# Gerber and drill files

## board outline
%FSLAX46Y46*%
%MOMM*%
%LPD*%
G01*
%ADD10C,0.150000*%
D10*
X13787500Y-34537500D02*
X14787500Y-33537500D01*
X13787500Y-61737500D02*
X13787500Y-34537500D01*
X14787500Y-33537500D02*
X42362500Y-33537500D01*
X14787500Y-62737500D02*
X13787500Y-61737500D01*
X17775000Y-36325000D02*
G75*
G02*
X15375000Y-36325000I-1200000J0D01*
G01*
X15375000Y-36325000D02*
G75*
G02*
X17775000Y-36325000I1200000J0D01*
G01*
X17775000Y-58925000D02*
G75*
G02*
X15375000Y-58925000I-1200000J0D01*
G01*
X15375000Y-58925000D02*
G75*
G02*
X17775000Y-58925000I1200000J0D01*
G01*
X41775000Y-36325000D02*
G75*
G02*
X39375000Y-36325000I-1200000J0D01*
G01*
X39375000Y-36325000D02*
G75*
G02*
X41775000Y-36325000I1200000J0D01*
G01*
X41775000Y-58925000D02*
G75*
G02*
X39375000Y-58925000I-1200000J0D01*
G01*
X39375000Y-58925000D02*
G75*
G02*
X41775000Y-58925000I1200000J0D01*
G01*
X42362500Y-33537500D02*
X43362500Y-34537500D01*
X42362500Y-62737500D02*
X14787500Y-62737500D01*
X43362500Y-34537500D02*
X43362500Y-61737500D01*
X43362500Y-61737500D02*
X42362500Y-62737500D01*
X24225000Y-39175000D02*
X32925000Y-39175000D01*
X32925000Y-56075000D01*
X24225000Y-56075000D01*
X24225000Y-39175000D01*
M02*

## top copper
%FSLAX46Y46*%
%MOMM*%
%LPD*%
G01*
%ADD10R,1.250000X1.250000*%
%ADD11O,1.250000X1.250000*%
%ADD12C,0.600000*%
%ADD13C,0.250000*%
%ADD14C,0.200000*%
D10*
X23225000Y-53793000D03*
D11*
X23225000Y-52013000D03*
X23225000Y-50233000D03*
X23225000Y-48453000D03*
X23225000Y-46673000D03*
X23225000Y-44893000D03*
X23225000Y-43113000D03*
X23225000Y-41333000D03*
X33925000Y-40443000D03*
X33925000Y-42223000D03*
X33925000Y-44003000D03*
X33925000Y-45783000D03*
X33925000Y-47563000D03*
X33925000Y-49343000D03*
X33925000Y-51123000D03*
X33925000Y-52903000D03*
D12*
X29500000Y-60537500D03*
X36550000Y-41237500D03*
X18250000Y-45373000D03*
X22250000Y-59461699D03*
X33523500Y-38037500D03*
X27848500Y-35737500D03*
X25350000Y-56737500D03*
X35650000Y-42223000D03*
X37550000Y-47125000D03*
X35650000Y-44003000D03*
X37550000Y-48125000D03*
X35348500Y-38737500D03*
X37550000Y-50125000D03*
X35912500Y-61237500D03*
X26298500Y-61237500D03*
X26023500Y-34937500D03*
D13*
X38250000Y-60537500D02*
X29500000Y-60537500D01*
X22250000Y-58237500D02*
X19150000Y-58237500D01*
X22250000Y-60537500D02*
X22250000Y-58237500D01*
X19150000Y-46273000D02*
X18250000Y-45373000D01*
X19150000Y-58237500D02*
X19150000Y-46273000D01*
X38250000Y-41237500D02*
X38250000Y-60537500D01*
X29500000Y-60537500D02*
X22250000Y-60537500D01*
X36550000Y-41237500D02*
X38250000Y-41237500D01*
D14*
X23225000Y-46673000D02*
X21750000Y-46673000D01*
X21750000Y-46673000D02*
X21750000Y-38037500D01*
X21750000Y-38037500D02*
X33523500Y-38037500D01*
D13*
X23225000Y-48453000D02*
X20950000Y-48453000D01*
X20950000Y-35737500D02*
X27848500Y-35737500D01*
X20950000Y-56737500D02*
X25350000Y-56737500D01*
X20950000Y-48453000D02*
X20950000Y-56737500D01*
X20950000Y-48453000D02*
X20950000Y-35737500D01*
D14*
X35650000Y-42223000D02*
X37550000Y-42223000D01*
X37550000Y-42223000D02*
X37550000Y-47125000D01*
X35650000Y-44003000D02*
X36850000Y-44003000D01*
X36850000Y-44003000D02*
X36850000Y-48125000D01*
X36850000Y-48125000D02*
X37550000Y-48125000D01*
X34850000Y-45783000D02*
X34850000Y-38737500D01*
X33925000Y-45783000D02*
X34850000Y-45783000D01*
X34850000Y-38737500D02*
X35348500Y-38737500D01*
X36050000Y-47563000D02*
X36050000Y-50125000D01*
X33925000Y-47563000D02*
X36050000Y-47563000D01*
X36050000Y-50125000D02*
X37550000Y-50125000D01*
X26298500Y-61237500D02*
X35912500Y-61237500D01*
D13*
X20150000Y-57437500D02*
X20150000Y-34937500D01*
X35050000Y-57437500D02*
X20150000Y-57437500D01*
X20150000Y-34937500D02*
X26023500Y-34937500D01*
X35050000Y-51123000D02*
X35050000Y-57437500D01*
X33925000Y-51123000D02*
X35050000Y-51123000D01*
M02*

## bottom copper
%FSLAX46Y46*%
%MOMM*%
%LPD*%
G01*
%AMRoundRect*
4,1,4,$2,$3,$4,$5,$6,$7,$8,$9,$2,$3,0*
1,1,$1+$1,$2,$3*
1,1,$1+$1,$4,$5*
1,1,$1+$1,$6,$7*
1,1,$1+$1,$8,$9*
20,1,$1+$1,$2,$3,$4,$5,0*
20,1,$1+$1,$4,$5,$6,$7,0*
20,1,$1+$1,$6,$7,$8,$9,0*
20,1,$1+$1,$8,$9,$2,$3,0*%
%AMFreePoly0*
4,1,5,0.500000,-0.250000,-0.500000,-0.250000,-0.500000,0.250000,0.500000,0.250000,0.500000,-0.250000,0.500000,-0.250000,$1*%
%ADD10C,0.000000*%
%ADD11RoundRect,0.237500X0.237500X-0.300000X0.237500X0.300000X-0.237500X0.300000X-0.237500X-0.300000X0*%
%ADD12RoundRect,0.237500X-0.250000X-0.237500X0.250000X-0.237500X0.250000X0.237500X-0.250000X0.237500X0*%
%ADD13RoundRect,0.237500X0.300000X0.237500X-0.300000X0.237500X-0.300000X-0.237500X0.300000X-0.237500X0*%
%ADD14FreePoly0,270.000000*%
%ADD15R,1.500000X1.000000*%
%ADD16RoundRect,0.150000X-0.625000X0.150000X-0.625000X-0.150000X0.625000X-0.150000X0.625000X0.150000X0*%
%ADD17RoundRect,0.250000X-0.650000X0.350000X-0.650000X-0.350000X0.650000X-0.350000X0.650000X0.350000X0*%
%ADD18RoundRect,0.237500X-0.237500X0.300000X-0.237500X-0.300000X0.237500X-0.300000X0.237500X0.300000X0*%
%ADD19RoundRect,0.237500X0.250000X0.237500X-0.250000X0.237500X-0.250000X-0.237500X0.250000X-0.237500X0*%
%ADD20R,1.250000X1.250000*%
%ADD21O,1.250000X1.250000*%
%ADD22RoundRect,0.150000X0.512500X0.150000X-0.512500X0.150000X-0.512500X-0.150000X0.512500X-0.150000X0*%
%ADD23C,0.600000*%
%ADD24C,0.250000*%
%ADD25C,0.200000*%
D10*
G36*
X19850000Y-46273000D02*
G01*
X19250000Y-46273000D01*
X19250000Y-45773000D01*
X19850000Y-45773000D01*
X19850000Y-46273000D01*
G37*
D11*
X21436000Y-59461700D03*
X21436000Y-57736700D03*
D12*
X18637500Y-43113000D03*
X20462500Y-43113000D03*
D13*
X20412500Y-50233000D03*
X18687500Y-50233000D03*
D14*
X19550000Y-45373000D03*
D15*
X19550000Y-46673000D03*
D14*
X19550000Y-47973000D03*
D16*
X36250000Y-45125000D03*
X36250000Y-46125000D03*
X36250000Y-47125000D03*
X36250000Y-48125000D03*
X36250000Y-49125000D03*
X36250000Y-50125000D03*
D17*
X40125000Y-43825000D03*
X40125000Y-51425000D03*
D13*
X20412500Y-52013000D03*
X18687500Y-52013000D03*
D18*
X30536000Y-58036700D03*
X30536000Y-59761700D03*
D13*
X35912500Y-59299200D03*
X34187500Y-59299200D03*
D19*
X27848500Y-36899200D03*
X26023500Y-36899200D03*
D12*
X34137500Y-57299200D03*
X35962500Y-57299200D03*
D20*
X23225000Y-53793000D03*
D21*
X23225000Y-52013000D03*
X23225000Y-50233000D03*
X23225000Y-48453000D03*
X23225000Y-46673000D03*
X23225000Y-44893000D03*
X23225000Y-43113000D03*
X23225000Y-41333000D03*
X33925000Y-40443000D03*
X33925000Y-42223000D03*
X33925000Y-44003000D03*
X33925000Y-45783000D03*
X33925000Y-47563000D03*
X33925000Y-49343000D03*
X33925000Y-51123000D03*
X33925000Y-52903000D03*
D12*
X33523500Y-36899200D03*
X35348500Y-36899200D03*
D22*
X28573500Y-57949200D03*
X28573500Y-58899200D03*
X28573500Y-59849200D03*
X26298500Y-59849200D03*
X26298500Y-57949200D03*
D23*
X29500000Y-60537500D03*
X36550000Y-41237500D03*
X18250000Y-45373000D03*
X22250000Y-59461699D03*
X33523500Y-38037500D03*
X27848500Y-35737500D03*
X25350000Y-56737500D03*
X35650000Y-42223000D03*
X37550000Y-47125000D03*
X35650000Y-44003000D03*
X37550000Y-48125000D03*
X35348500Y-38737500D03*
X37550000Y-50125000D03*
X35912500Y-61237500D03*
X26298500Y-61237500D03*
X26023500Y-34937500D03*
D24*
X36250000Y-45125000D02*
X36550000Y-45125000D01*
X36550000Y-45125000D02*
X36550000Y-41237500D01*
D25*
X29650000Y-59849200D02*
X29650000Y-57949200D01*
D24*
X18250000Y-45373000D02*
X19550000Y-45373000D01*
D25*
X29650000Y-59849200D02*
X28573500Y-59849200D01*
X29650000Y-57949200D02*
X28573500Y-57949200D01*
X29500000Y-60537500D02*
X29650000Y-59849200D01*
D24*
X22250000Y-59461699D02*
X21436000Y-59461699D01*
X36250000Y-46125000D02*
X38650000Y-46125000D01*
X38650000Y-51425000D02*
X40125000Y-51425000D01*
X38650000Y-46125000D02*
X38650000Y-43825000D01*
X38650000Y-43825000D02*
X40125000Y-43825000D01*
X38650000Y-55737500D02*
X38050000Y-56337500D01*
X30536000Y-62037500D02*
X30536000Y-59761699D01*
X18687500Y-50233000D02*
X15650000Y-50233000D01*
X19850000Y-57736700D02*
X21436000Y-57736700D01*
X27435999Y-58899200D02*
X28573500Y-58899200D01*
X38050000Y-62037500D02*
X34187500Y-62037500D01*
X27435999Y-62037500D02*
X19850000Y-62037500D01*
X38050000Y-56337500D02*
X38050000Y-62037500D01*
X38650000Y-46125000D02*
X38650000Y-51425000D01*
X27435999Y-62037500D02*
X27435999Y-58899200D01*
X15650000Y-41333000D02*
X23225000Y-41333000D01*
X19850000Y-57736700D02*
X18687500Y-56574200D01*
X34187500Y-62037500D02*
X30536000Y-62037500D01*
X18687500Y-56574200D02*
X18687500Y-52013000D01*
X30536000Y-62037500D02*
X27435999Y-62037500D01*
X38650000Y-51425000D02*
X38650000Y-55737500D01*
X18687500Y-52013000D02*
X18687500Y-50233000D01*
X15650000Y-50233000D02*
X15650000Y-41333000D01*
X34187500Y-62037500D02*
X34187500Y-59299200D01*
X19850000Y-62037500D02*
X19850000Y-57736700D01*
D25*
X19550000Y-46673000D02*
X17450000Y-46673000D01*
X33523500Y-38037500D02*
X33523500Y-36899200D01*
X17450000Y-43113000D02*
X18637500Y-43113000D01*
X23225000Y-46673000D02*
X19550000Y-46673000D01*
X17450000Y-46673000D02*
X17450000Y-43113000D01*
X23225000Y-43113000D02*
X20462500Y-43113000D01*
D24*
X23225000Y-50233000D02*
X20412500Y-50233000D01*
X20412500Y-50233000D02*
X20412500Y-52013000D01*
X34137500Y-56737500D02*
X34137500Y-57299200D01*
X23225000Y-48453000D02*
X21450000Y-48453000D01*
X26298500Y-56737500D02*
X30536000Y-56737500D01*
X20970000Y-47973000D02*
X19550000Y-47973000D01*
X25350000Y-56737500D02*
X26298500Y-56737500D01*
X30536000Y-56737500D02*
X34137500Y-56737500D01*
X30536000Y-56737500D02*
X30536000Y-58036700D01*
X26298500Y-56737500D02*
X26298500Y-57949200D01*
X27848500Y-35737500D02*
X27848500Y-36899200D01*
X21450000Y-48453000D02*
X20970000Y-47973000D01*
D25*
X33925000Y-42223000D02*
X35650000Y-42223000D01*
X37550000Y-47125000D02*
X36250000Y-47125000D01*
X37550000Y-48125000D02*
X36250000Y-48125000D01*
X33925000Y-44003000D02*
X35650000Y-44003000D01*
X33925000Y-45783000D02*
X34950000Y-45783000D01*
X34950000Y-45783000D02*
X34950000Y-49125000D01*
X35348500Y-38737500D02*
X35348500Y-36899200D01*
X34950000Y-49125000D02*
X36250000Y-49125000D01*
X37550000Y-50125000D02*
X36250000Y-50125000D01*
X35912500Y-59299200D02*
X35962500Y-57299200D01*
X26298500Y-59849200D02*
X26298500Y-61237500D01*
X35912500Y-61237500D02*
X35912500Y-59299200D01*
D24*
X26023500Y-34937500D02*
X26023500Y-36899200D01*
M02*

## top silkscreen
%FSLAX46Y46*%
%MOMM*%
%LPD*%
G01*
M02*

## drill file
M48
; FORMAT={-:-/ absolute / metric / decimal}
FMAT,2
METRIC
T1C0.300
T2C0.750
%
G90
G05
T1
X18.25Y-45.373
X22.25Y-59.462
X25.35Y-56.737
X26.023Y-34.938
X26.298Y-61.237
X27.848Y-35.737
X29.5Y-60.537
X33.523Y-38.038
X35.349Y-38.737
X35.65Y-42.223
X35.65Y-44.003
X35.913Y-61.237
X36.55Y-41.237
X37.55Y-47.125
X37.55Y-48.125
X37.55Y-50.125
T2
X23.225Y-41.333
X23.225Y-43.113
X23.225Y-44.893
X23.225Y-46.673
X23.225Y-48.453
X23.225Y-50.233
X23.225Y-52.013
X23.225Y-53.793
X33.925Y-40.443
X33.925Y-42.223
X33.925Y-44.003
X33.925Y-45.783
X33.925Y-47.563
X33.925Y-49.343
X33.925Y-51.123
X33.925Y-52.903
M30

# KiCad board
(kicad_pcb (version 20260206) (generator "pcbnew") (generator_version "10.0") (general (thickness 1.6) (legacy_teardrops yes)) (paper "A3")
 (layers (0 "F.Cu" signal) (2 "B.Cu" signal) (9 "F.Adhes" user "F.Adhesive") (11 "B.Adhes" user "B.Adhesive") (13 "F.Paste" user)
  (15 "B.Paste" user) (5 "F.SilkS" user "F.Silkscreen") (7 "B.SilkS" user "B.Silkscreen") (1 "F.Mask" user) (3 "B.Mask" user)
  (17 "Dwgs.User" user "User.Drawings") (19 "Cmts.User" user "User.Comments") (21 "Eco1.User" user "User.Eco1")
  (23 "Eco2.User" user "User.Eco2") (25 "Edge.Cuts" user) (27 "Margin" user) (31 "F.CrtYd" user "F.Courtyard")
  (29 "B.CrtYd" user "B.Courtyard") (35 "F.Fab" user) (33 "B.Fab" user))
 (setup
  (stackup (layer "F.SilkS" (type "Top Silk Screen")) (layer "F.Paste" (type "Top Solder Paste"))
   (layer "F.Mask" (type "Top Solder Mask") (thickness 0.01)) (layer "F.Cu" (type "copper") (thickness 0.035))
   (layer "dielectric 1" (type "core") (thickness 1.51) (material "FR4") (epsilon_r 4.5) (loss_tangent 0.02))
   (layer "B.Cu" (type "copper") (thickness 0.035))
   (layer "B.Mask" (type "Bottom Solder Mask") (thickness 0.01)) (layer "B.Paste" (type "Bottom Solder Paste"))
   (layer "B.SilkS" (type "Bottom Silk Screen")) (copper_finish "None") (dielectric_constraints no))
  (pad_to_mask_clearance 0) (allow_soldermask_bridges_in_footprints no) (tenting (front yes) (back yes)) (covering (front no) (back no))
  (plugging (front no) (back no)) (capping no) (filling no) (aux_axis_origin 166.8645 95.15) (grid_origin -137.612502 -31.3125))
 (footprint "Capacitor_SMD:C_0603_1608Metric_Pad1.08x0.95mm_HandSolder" (layer "B.Cu") (at 21.436 58.5992 90)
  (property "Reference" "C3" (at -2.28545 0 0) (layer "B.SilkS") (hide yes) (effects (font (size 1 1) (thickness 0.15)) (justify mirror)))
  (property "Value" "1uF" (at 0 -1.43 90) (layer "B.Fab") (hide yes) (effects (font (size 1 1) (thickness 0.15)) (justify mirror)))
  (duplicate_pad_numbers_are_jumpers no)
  (pad "1" smd roundrect (at -0.8625 0 90) (size 1.075 0.95) (layers "B.Cu" "B.Mask" "B.Paste") (roundrect_rratio 0.25) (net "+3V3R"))
  (pad "2" smd roundrect (at 0.8625 0 90) (size 1.075 0.95) (layers "B.Cu" "B.Mask" "B.Paste") (roundrect_rratio 0.25) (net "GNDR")))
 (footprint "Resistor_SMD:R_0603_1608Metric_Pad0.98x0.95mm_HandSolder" (layer "B.Cu") (at 19.55 43.113)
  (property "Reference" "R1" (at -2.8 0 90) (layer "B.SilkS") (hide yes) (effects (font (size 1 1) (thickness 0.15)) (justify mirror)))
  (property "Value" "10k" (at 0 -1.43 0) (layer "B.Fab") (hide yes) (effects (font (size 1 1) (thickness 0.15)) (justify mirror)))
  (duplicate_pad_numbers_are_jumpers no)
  (pad "1" smd roundrect (at -0.9125 0) (size 0.975 0.95) (layers "B.Cu" "B.Mask" "B.Paste") (roundrect_rratio 0.25) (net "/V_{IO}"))
  (pad "2" smd roundrect (at 0.9125 0) (size 0.975 0.95) (layers "B.Cu" "B.Mask" "B.Paste") (roundrect_rratio 0.25) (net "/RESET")))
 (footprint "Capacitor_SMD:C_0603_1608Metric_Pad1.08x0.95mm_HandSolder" (layer "B.Cu") (at 19.55 50.233 180)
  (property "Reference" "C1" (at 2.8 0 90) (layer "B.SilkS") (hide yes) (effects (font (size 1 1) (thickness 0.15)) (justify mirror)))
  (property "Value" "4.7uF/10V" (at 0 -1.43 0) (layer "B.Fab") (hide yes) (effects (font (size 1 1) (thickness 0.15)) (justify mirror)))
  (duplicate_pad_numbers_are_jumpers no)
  (pad "1" smd roundrect (at -0.8625 0 180) (size 1.075 0.95) (layers "B.Cu" "B.Mask" "B.Paste") (roundrect_rratio 0.25)
   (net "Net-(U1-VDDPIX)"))
  (pad "2" smd roundrect (at 0.8625 0 180) (size 1.075 0.95) (layers "B.Cu" "B.Mask" "B.Paste") (roundrect_rratio 0.25) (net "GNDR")))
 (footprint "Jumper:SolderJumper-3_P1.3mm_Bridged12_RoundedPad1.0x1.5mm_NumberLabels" (layer "B.Cu") (at 19.55 46.673 -90)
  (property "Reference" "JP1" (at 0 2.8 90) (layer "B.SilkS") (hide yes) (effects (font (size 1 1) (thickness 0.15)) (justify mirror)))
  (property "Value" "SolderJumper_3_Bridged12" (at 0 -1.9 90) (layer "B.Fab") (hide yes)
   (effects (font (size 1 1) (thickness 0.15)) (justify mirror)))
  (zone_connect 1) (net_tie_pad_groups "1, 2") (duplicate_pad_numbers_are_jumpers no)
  (fp_poly (pts (xy -0.9 0.3) (xy -0.4 0.3) (xy -0.4 -0.3) (xy -0.9 -0.3)) (stroke (width 0) (type solid)) (fill yes) (layer "B.Cu"))
  (pad "1" smd custom (at -1.3 0 270) (size 1 0.5) (layers "B.Cu" "B.Mask") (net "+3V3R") (zone_connect 2) (thermal_bridge_angle 45)
   (options (clearance outline) (anchor rect)) (primitives))
  (pad "2" smd rect (at 0 0 270) (size 1 1.5) (layers "B.Cu" "B.Mask") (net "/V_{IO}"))
  (pad "3" smd custom (at 1.3 0 270) (size 1 0.5) (layers "B.Cu" "B.Mask") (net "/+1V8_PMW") (zone_connect 2) (thermal_bridge_angle 45)
   (options (clearance outline) (anchor rect)) (primitives)))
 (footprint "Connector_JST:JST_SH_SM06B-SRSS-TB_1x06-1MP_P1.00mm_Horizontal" (layer "B.Cu") (at 38.25 47.625 -90)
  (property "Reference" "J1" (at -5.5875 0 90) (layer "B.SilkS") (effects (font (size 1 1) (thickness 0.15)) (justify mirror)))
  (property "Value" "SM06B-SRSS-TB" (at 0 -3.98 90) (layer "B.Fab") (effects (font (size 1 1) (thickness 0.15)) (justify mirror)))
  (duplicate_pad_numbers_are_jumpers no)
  (pad "1" smd roundrect (at -2.5 2 270) (size 0.6 1.55) (layers "B.Cu" "B.Mask" "B.Paste") (roundrect_rratio 0.25) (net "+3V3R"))
  (pad "2" smd roundrect (at -1.5 2 270) (size 0.6 1.55) (layers "B.Cu" "B.Mask" "B.Paste") (roundrect_rratio 0.25) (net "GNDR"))
  (pad "3" smd roundrect (at -0.5 2 270) (size 0.6 1.55) (layers "B.Cu" "B.Mask" "B.Paste") (roundrect_rratio 0.25) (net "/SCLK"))
  (pad "4" smd roundrect (at 0.5 2 270) (size 0.6 1.55) (layers "B.Cu" "B.Mask" "B.Paste") (roundrect_rratio 0.25) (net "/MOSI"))
  (pad "5" smd roundrect (at 1.5 2 270) (size 0.6 1.55) (layers "B.Cu" "B.Mask" "B.Paste") (roundrect_rratio 0.25) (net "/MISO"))
  (pad "6" smd roundrect (at 2.5 2 270) (size 0.6 1.55) (layers "B.Cu" "B.Mask" "B.Paste") (roundrect_rratio 0.25) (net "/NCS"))
  (pad "MP" smd roundrect (at -3.8 -1.875 270) (size 1.2 1.8) (layers "B.Cu" "B.Mask" "B.Paste") (roundrect_rratio 0.208333) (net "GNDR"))
  (pad "MP" smd roundrect (at 3.8 -1.875 270) (size 1.2 1.8) (layers "B.Cu" "B.Mask" "B.Paste") (roundrect_rratio 0.208333) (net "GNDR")))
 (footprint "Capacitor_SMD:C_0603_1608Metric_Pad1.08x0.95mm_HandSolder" (layer "B.Cu") (at 19.55 52.013 180)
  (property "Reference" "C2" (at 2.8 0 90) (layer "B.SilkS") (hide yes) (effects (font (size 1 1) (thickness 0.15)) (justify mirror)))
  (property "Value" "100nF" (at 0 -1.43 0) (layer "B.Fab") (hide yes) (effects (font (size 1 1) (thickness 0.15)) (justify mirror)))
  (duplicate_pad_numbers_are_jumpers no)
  (pad "1" smd roundrect (at -0.8625 0 180) (size 1.075 0.95) (layers "B.Cu" "B.Mask" "B.Paste") (roundrect_rratio 0.25)
   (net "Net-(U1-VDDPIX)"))
  (pad "2" smd roundrect (at 0.8625 0 180) (size 1.075 0.95) (layers "B.Cu" "B.Mask" "B.Paste") (roundrect_rratio 0.25) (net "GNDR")))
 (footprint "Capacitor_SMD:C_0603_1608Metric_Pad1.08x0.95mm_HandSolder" (layer "B.Cu") (at 30.536 58.8992 -90)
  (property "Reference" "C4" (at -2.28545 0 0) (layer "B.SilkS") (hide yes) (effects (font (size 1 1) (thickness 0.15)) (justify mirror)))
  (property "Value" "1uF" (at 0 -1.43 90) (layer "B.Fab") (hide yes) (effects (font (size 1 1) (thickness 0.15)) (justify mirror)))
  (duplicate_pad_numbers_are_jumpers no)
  (pad "1" smd roundrect (at -0.8625 0 270) (size 1.075 0.95) (layers "B.Cu" "B.Mask" "B.Paste") (roundrect_rratio 0.25) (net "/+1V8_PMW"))
  (pad "2" smd roundrect (at 0.8625 0 270) (size 1.075 0.95) (layers "B.Cu" "B.Mask" "B.Paste") (roundrect_rratio 0.25) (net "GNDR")))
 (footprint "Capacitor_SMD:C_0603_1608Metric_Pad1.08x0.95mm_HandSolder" (layer "B.Cu") (at 35.05 59.2992 180)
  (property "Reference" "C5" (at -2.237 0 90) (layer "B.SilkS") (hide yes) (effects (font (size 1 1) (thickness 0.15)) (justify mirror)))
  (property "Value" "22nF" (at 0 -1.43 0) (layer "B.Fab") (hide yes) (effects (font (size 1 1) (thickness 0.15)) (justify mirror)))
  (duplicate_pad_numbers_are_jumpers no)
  (pad "1" smd roundrect (at -0.8625 0 180) (size 1.075 0.95) (layers "B.Cu" "B.Mask" "B.Paste") (roundrect_rratio 0.25) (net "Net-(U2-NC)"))
  (pad "2" smd roundrect (at 0.8625 0 180) (size 1.075 0.95) (layers "B.Cu" "B.Mask" "B.Paste") (roundrect_rratio 0.25) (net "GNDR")))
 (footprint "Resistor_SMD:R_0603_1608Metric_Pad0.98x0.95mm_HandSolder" (layer "B.Cu") (at 26.936 36.8992 180)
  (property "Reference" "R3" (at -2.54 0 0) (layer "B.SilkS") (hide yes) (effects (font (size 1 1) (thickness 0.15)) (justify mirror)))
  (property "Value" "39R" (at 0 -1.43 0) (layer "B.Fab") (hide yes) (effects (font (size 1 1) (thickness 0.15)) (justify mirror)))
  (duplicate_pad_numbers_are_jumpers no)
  (pad "1" smd roundrect (at -0.9125 0 180) (size 0.975 0.95) (layers "B.Cu" "B.Mask" "B.Paste") (roundrect_rratio 0.25) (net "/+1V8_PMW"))
  (pad "2" smd roundrect (at 0.9125 0 180) (size 0.975 0.95) (layers "B.Cu" "B.Mask" "B.Paste") (roundrect_rratio 0.25)
   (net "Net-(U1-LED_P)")))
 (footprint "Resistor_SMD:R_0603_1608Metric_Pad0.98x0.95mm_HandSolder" (layer "B.Cu") (at 35.05 57.2992)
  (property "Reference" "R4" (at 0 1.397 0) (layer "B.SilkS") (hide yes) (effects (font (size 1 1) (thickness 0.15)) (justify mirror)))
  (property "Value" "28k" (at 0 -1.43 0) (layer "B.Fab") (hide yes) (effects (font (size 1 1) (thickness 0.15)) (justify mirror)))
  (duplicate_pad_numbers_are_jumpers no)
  (pad "1" smd roundrect (at -0.9125 0) (size 0.975 0.95) (layers "B.Cu" "B.Mask" "B.Paste") (roundrect_rratio 0.25) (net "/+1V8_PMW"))
  (pad "2" smd roundrect (at 0.9125 0) (size 0.975 0.95) (layers "B.Cu" "B.Mask" "B.Paste") (roundrect_rratio 0.25) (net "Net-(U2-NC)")))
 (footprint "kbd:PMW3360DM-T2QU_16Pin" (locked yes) (layer "B.Cu") (at 28.575 47.625 90)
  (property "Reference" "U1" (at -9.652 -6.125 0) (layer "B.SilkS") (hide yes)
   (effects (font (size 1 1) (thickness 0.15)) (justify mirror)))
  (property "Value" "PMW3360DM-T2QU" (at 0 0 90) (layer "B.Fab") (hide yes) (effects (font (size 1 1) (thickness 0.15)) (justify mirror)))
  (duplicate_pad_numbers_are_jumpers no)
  (fp_rect (start 8.45 4.35) (end -8.45 -4.35) (stroke (width 0.15) (type solid)) (fill no) (layer "Edge.Cuts"))
  (pad "1" thru_hole rect (at -6.168 -5.35 90) (size 1.25 1.25) (drill 0.75) (layers "*.Cu" "*.Mask") (remove_unused_layers no)
   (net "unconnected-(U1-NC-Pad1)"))
  (pad "2" thru_hole oval (at -4.388 -5.35 90) (size 1.25 1.25) (drill 0.75) (layers "*.Cu" "*.Mask") (remove_unused_layers no)
   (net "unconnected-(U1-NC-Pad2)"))
  (pad "3" thru_hole oval (at -2.608 -5.35 90) (size 1.25 1.25) (drill 0.75) (layers "*.Cu" "*.Mask") (remove_unused_layers no)
   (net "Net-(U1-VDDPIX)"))
  (pad "4" thru_hole oval (at -0.828 -5.35 90) (size 1.25 1.25) (drill 0.75) (layers "*.Cu" "*.Mask") (remove_unused_layers no)
   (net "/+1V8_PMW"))
  (pad "5" thru_hole oval (at 0.952 -5.35 90) (size 1.25 1.25) (drill 0.75) (layers "*.Cu" "*.Mask") (remove_unused_layers no)
   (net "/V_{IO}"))
  (pad "6" thru_hole oval (at 2.732 -5.35 90) (size 1.25 1.25) (drill 0.75) (layers "*.Cu" "*.Mask") (remove_unused_layers no)
   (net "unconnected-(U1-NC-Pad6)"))
  (pad "7" thru_hole oval (at 4.512 -5.35 90) (size 1.25 1.25) (drill 0.75) (layers "*.Cu" "*.Mask") (remove_unused_layers no)
   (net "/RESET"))
  (pad "8" thru_hole oval (at 6.292 -5.35 90) (size 1.25 1.25) (drill 0.75) (layers "*.Cu" "*.Mask") (remove_unused_layers no) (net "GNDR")
   (zone_connect 2))
  (pad "9" thru_hole oval (at 7.182 5.35 90) (size 1.25 1.25) (drill 0.75) (layers "*.Cu" "*.Mask") (remove_unused_layers no)
   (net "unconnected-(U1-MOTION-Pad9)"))
  (pad "10" thru_hole oval (at 5.402 5.35 90) (size 1.25 1.25) (drill 0.75) (layers "*.Cu" "*.Mask") (remove_unused_layers no) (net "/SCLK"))
  (pad "11" thru_hole oval (at 3.622 5.35 90) (size 1.25 1.25) (drill 0.75) (layers "*.Cu" "*.Mask") (remove_unused_layers no) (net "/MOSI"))
  (pad "12" thru_hole oval (at 1.842 5.35 90) (size 1.25 1.25) (drill 0.75) (layers "*.Cu" "*.Mask") (remove_unused_layers no) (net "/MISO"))
  (pad "13" thru_hole oval (at 0.062 5.35 90) (size 1.25 1.25) (drill 0.75) (layers "*.Cu" "*.Mask") (remove_unused_layers no) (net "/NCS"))
  (pad "14" thru_hole oval (at -1.718 5.35 90) (size 1.25 1.25) (drill 0.75) (layers "*.Cu" "*.Mask") (remove_unused_layers no)
   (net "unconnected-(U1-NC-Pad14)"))
  (pad "15" thru_hole oval (at -3.498 5.35 90) (size 1.25 1.25) (drill 0.75) (layers "*.Cu" "*.Mask") (remove_unused_layers no)
   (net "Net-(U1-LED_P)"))
  (pad "16" thru_hole oval (at -5.278 5.35 90) (size 1.25 1.25) (drill 0.75) (layers "*.Cu" "*.Mask") (remove_unused_layers no)
   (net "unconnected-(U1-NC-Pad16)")))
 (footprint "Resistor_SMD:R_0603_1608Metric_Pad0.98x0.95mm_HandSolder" (layer "B.Cu") (at 34.436 36.8992)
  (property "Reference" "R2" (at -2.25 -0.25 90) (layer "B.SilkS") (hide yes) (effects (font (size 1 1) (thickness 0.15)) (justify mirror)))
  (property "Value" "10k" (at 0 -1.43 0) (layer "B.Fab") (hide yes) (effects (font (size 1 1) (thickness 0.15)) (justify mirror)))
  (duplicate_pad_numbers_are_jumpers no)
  (pad "1" smd roundrect (at -0.9125 0) (size 0.975 0.95) (layers "B.Cu" "B.Mask" "B.Paste") (roundrect_rratio 0.25) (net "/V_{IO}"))
  (pad "2" smd roundrect (at 0.9125 0) (size 0.975 0.95) (layers "B.Cu" "B.Mask" "B.Paste") (roundrect_rratio 0.25) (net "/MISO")))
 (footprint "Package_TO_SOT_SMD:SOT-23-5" (layer "B.Cu") (at 27.436 58.8992 180)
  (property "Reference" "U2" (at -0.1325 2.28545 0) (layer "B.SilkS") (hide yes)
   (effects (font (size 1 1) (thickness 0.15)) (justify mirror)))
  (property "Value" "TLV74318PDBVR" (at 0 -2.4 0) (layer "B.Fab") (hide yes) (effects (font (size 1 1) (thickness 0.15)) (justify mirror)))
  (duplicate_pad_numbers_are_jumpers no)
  (pad "1" smd roundrect (at -1.1375 0.95 180) (size 1.325 0.6) (layers "B.Cu" "B.Mask" "B.Paste") (roundrect_rratio 0.25) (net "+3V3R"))
  (pad "2" smd roundrect (at -1.1375 0 180) (size 1.325 0.6) (layers "B.Cu" "B.Mask" "B.Paste") (roundrect_rratio 0.25) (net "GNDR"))
  (pad "3" smd roundrect (at -1.1375 -0.95 180) (size 1.325 0.6) (layers "B.Cu" "B.Mask" "B.Paste") (roundrect_rratio 0.25) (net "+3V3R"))
  (pad "4" smd roundrect (at 1.1375 -0.95 180) (size 1.325 0.6) (layers "B.Cu" "B.Mask" "B.Paste") (roundrect_rratio 0.25)
   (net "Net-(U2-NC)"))
  (pad "5" smd roundrect (at 1.1375 0.95 180) (size 1.325 0.6) (layers "B.Cu" "B.Mask" "B.Paste") (roundrect_rratio 0.25) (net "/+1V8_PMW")))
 (gr_line (start 13.7875 34.5375) (end 14.7875 33.5375) (stroke (width 0.15) (type default)) (layer "Edge.Cuts"))
 (gr_line (start 13.7875 61.7375) (end 13.7875 34.5375) (stroke (width 0.15) (type default)) (layer "Edge.Cuts"))
 (gr_line (start 14.7875 33.5375) (end 42.3625 33.5375) (stroke (width 0.15) (type default)) (layer "Edge.Cuts"))
 (gr_line (start 14.7875 62.7375) (end 13.7875 61.7375) (stroke (width 0.15) (type default)) (layer "Edge.Cuts"))
 (gr_circle (center 16.575 36.325) (end 17.775 36.325) (stroke (width 0.15) (type default)) (fill no) (layer "Edge.Cuts"))
 (gr_circle (center 16.575 58.925) (end 17.775 58.925) (stroke (width 0.15) (type default)) (fill no) (layer "Edge.Cuts"))
 (gr_circle (center 40.575 36.325) (end 41.775 36.325) (stroke (width 0.15) (type default)) (fill no) (layer "Edge.Cuts"))
 (gr_circle (center 40.575 58.925) (end 41.775 58.925) (stroke (width 0.15) (type default)) (fill no) (layer "Edge.Cuts"))
 (gr_line (start 42.3625 33.5375) (end 43.3625 34.5375) (stroke (width 0.15) (type default)) (layer "Edge.Cuts"))
 (gr_line (start 42.3625 62.7375) (end 14.7875 62.7375) (stroke (width 0.15) (type default)) (layer "Edge.Cuts"))
 (gr_line (start 43.3625 34.5375) (end 43.3625 61.7375) (stroke (width 0.15) (type default)) (layer "Edge.Cuts"))
 (gr_line (start 43.3625 61.7375) (end 42.3625 62.7375) (stroke (width 0.15) (type default)) (layer "Edge.Cuts"))
 (segment (start 38.25 60.5375) (end 29.5 60.5375) (width 0.25) (layer "F.Cu") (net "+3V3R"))
 (segment (start 22.25 58.2375) (end 19.15 58.2375) (width 0.25) (layer "F.Cu") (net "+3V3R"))
 (segment (start 22.25 60.5375) (end 22.25 58.2375) (width 0.25) (layer "F.Cu") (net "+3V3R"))
 (segment (start 19.15 46.273) (end 18.25 45.373) (width 0.25) (layer "F.Cu") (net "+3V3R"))
 (segment (start 19.15 58.2375) (end 19.15 46.273) (width 0.25) (layer "F.Cu") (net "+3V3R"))
 (segment (start 38.25 41.2375) (end 38.25 60.5375) (width 0.25) (layer "F.Cu") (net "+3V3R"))
 (segment (start 29.5 60.5375) (end 22.25 60.5375) (width 0.25) (layer "F.Cu") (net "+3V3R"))
 (segment (start 36.55 41.2375) (end 38.25 41.2375) (width 0.25) (layer "F.Cu") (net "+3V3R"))
 (via (at 29.5 60.5375) (size 0.6) (drill 0.3) (layers "F.Cu" "B.Cu") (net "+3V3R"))
 (via (at 36.55 41.2375) (size 0.6) (drill 0.3) (layers "F.Cu" "B.Cu") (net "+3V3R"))
 (via (at 18.25 45.373) (size 0.6) (drill 0.3) (layers "F.Cu" "B.Cu") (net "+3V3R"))
 (via (at 22.25 59.461699) (size 0.6) (drill 0.3) (layers "F.Cu" "B.Cu") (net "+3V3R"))
 (segment (start 36.25 45.125) (end 36.55 45.125) (width 0.25) (layer "B.Cu") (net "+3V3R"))
 (segment (start 36.55 45.125) (end 36.55 41.2375) (width 0.25) (layer "B.Cu") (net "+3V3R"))
 (segment (start 29.65 59.8492) (end 29.65 57.9492) (width 0.2) (layer "B.Cu") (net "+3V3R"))
 (segment (start 18.25 45.373) (end 19.55 45.373) (width 0.25) (layer "B.Cu") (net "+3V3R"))
 (segment (start 29.65 59.8492) (end 28.5735 59.8492) (width 0.2) (layer "B.Cu") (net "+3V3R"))
 (segment (start 29.65 57.9492) (end 28.5735 57.9492) (width 0.2) (layer "B.Cu") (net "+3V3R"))
 (segment (start 29.5 60.5375) (end 29.65 59.8492) (width 0.2) (layer "B.Cu") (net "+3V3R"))
 (segment (start 22.25 59.461699) (end 21.436 59.461699) (width 0.25) (layer "B.Cu") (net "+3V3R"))
 (segment (start 36.25 46.125) (end 38.65 46.125) (width 0.25) (layer "B.Cu") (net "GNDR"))
 (segment (start 38.65 51.425) (end 40.125 51.425) (width 0.25) (layer "B.Cu") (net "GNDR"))
 (segment (start 38.65 46.125) (end 38.65 43.825) (width 0.25) (layer "B.Cu") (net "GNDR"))
 (segment (start 38.65 43.825) (end 40.125 43.825) (width 0.25) (layer "B.Cu") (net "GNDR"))
 (segment (start 38.65 55.7375) (end 38.05 56.3375) (width 0.25) (layer "B.Cu") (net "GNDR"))
 (segment (start 30.536 62.0375) (end 30.536 59.761699) (width 0.25) (layer "B.Cu") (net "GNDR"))
 (segment (start 18.6875 50.233) (end 15.65 50.233) (width 0.25) (layer "B.Cu") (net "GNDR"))
 (segment (start 19.85 57.7367) (end 21.436 57.7367) (width 0.25) (layer "B.Cu") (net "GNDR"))
 (segment (start 27.435999 58.8992) (end 28.5735 58.8992) (width 0.25) (layer "B.Cu") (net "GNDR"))
 (segment (start 38.05 62.0375) (end 34.1875 62.0375) (width 0.25) (layer "B.Cu") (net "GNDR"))
 (segment (start 27.435999 62.0375) (end 19.85 62.0375) (width 0.25) (layer "B.Cu") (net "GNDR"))
 (segment (start 38.05 56.3375) (end 38.05 62.0375) (width 0.25) (layer "B.Cu") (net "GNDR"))
 (segment (start 38.65 46.125) (end 38.65 51.425) (width 0.25) (layer "B.Cu") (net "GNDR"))
 (segment (start 27.435999 62.0375) (end 27.435999 58.8992) (width 0.25) (layer "B.Cu") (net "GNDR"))
 (segment (start 15.65 41.333) (end 23.225 41.333) (width 0.25) (layer "B.Cu") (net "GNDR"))
 (segment (start 19.85 57.7367) (end 18.6875 56.5742) (width 0.25) (layer "B.Cu") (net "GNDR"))
 (segment (start 34.1875 62.0375) (end 30.536 62.0375) (width 0.25) (layer "B.Cu") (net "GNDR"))
 (segment (start 18.6875 56.5742) (end 18.6875 52.013) (width 0.25) (layer "B.Cu") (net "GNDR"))
 (segment (start 30.536 62.0375) (end 27.435999 62.0375) (width 0.25) (layer "B.Cu") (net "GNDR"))
 (segment (start 38.65 51.425) (end 38.65 55.7375) (width 0.25) (layer "B.Cu") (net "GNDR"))
 (segment (start 18.6875 52.013) (end 18.6875 50.233) (width 0.25) (layer "B.Cu") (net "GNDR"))
 (segment (start 15.65 50.233) (end 15.65 41.333) (width 0.25) (layer "B.Cu") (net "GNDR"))
 (segment (start 34.1875 62.0375) (end 34.1875 59.2992) (width 0.25) (layer "B.Cu") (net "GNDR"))
 (segment (start 19.85 62.0375) (end 19.85 57.7367) (width 0.25) (layer "B.Cu") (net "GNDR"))
 (segment (start 23.225 46.673) (end 21.75 46.673) (width 0.2) (layer "F.Cu") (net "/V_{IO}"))
 (segment (start 21.75 46.673) (end 21.75 38.0375) (width 0.2) (layer "F.Cu") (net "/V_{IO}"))
 (segment (start 21.75 38.0375) (end 33.5235 38.0375) (width 0.2) (layer "F.Cu") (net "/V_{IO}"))
 (via (at 33.5235 38.0375) (size 0.6) (drill 0.3) (layers "F.Cu" "B.Cu") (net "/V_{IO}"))
 (segment (start 19.55 46.673) (end 17.45 46.673) (width 0.2) (layer "B.Cu") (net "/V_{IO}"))
 (segment (start 33.5235 38.0375) (end 33.5235 36.8992) (width 0.2) (layer "B.Cu") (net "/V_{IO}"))
 (segment (start 17.45 43.113) (end 18.6375 43.113) (width 0.2) (layer "B.Cu") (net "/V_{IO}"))
 (segment (start 23.225 46.673) (end 19.55 46.673) (width 0.2) (layer "B.Cu") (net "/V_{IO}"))
 (segment (start 17.45 46.673) (end 17.45 43.113) (width 0.2) (layer "B.Cu") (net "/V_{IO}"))
 (segment (start 23.225 43.113) (end 20.4625 43.113) (width 0.2) (layer "B.Cu") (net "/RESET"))
 (segment (start 23.225 50.233) (end 20.4125 50.233) (width 0.25) (layer "B.Cu") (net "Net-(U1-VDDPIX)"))
 (segment (start 20.4125 50.233) (end 20.4125 52.013) (width 0.25) (layer "B.Cu") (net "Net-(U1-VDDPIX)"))
 (segment (start 23.225 48.453) (end 20.95 48.453) (width 0.25) (layer "F.Cu") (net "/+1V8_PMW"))
 (segment (start 20.95 35.7375) (end 27.8485 35.7375) (width 0.25) (layer "F.Cu") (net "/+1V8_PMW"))
 (segment (start 20.95 56.7375) (end 25.35 56.7375) (width 0.25) (layer "F.Cu") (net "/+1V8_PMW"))
 (segment (start 20.95 48.453) (end 20.95 56.7375) (width 0.25) (layer "F.Cu") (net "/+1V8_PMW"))
 (segment (start 20.95 48.453) (end 20.95 35.7375) (width 0.25) (layer "F.Cu") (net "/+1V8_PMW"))
 (via (at 27.8485 35.7375) (size 0.6) (drill 0.3) (layers "F.Cu" "B.Cu") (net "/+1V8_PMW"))
 (via (at 25.35 56.7375) (size 0.6) (drill 0.3) (layers "F.Cu" "B.Cu") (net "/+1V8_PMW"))
 (segment (start 34.1375 56.7375) (end 34.1375 57.2992) (width 0.25) (layer "B.Cu") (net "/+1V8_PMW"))
 (segment (start 23.225 48.453) (end 21.45 48.453) (width 0.25) (layer "B.Cu") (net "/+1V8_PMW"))
 (segment (start 26.2985 56.7375) (end 30.536 56.7375) (width 0.25) (layer "B.Cu") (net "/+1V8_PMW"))
 (segment (start 20.97 47.973) (end 19.55 47.973) (width 0.25) (layer "B.Cu") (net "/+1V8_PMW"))
 (segment (start 25.35 56.7375) (end 26.2985 56.7375) (width 0.25) (layer "B.Cu") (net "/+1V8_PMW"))
 (segment (start 30.536 56.7375) (end 34.1375 56.7375) (width 0.25) (layer "B.Cu") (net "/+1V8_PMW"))
 (segment (start 30.536 56.7375) (end 30.536 58.0367) (width 0.25) (layer "B.Cu") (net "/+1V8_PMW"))
 (segment (start 26.2985 56.7375) (end 26.2985 57.9492) (width 0.25) (layer "B.Cu") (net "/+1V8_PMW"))
 (segment (start 27.8485 35.7375) (end 27.8485 36.8992) (width 0.25) (layer "B.Cu") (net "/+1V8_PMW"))
 (segment (start 21.45 48.453) (end 20.97 47.973) (width 0.25) (layer "B.Cu") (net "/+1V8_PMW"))
 (segment (start 35.65 42.223) (end 37.55 42.223) (width 0.2) (layer "F.Cu") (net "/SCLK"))
 (segment (start 37.55 42.223) (end 37.55 47.125) (width 0.2) (layer "F.Cu") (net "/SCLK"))
 (via (at 35.65 42.223) (size 0.6) (drill 0.3) (layers "F.Cu" "B.Cu") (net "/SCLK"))
 (via (at 37.55 47.125) (size 0.6) (drill 0.3) (layers "F.Cu" "B.Cu") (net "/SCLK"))
 (segment (start 33.925 42.223) (end 35.65 42.223) (width 0.2) (layer "B.Cu") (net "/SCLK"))
 (segment (start 37.55 47.125) (end 36.25 47.125) (width 0.2) (layer "B.Cu") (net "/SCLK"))
 (segment (start 35.65 44.003) (end 36.85 44.003) (width 0.2) (layer "F.Cu") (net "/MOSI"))
 (segment (start 36.85 44.003) (end 36.85 48.125) (width 0.2) (layer "F.Cu") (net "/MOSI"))
 (segment (start 36.85 48.125) (end 37.55 48.125) (width 0.2) (layer "F.Cu") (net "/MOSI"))
 (via (at 35.65 44.003) (size 0.6) (drill 0.3) (layers "F.Cu" "B.Cu") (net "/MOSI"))
 (via (at 37.55 48.125) (size 0.6) (drill 0.3) (layers "F.Cu" "B.Cu") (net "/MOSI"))
 (segment (start 37.55 48.125) (end 36.25 48.125) (width 0.2) (layer "B.Cu") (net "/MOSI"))
 (segment (start 33.925 44.003) (end 35.65 44.003) (width 0.2) (layer "B.Cu") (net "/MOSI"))
 (segment (start 34.85 45.783) (end 34.85 38.7375) (width 0.2) (layer "F.Cu") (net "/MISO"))
 (segment (start 33.925 45.783) (end 34.85 45.783) (width 0.2) (layer "F.Cu") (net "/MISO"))
 (segment (start 34.85 38.7375) (end 35.3485 38.7375) (width 0.2) (layer "F.Cu") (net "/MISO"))
 (via (at 35.3485 38.7375) (size 0.6) (drill 0.3) (layers "F.Cu" "B.Cu") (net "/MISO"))
 (segment (start 33.925 45.783) (end 34.95 45.783) (width 0.2) (layer "B.Cu") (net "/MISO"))
 (segment (start 34.95 45.783) (end 34.95 49.125) (width 0.2) (layer "B.Cu") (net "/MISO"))
 (segment (start 35.3485 38.7375) (end 35.3485 36.8992) (width 0.2) (layer "B.Cu") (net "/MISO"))
 (segment (start 34.95 49.125) (end 36.25 49.125) (width 0.2) (layer "B.Cu") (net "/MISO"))
 (segment (start 36.05 47.563) (end 36.05 50.125) (width 0.2) (layer "F.Cu") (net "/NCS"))
 (segment (start 33.925 47.563) (end 36.05 47.563) (width 0.2) (layer "F.Cu") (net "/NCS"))
 (segment (start 36.05 50.125) (end 37.55 50.125) (width 0.2) (layer "F.Cu") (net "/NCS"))
 (via (at 37.55 50.125) (size 0.6) (drill 0.3) (layers "F.Cu" "B.Cu") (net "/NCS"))
 (segment (start 37.55 50.125) (end 36.25 50.125) (width 0.2) (layer "B.Cu") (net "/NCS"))
 (segment (start 26.2985 61.2375) (end 35.9125 61.2375) (width 0.2) (layer "F.Cu") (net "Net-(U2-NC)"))
 (via (at 35.9125 61.2375) (size 0.6) (drill 0.3) (layers "F.Cu" "B.Cu") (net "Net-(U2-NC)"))
 (via (at 26.2985 61.2375) (size 0.6) (drill 0.3) (layers "F.Cu" "B.Cu") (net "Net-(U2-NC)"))
 (segment (start 35.9125 59.2992) (end 35.9625 57.2992) (width 0.2) (layer "B.Cu") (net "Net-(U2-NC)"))
 (segment (start 26.2985 59.8492) (end 26.2985 61.2375) (width 0.2) (layer "B.Cu") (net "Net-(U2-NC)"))
 (segment (start 35.9125 61.2375) (end 35.9125 59.2992) (width 0.2) (layer "B.Cu") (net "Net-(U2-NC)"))
 (segment (start 20.15 57.4375) (end 20.15 34.9375) (width 0.25) (layer "F.Cu") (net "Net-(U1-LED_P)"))
 (segment (start 35.05 57.4375) (end 20.15 57.4375) (width 0.25) (layer "F.Cu") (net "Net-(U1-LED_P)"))
 (segment (start 20.15 34.9375) (end 26.0235 34.9375) (width 0.25) (layer "F.Cu") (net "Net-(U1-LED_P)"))
 (segment (start 35.05 51.123) (end 35.05 57.4375) (width 0.25) (layer "F.Cu") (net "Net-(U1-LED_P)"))
 (segment (start 33.925 51.123) (end 35.05 51.123) (width 0.25) (layer "F.Cu") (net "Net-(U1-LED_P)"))
 (via (at 26.0235 34.9375) (size 0.6) (drill 0.3) (layers "F.Cu" "B.Cu") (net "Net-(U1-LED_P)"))
 (segment (start 26.0235 34.9375) (end 26.0235 36.8992) (width 0.25) (layer "B.Cu") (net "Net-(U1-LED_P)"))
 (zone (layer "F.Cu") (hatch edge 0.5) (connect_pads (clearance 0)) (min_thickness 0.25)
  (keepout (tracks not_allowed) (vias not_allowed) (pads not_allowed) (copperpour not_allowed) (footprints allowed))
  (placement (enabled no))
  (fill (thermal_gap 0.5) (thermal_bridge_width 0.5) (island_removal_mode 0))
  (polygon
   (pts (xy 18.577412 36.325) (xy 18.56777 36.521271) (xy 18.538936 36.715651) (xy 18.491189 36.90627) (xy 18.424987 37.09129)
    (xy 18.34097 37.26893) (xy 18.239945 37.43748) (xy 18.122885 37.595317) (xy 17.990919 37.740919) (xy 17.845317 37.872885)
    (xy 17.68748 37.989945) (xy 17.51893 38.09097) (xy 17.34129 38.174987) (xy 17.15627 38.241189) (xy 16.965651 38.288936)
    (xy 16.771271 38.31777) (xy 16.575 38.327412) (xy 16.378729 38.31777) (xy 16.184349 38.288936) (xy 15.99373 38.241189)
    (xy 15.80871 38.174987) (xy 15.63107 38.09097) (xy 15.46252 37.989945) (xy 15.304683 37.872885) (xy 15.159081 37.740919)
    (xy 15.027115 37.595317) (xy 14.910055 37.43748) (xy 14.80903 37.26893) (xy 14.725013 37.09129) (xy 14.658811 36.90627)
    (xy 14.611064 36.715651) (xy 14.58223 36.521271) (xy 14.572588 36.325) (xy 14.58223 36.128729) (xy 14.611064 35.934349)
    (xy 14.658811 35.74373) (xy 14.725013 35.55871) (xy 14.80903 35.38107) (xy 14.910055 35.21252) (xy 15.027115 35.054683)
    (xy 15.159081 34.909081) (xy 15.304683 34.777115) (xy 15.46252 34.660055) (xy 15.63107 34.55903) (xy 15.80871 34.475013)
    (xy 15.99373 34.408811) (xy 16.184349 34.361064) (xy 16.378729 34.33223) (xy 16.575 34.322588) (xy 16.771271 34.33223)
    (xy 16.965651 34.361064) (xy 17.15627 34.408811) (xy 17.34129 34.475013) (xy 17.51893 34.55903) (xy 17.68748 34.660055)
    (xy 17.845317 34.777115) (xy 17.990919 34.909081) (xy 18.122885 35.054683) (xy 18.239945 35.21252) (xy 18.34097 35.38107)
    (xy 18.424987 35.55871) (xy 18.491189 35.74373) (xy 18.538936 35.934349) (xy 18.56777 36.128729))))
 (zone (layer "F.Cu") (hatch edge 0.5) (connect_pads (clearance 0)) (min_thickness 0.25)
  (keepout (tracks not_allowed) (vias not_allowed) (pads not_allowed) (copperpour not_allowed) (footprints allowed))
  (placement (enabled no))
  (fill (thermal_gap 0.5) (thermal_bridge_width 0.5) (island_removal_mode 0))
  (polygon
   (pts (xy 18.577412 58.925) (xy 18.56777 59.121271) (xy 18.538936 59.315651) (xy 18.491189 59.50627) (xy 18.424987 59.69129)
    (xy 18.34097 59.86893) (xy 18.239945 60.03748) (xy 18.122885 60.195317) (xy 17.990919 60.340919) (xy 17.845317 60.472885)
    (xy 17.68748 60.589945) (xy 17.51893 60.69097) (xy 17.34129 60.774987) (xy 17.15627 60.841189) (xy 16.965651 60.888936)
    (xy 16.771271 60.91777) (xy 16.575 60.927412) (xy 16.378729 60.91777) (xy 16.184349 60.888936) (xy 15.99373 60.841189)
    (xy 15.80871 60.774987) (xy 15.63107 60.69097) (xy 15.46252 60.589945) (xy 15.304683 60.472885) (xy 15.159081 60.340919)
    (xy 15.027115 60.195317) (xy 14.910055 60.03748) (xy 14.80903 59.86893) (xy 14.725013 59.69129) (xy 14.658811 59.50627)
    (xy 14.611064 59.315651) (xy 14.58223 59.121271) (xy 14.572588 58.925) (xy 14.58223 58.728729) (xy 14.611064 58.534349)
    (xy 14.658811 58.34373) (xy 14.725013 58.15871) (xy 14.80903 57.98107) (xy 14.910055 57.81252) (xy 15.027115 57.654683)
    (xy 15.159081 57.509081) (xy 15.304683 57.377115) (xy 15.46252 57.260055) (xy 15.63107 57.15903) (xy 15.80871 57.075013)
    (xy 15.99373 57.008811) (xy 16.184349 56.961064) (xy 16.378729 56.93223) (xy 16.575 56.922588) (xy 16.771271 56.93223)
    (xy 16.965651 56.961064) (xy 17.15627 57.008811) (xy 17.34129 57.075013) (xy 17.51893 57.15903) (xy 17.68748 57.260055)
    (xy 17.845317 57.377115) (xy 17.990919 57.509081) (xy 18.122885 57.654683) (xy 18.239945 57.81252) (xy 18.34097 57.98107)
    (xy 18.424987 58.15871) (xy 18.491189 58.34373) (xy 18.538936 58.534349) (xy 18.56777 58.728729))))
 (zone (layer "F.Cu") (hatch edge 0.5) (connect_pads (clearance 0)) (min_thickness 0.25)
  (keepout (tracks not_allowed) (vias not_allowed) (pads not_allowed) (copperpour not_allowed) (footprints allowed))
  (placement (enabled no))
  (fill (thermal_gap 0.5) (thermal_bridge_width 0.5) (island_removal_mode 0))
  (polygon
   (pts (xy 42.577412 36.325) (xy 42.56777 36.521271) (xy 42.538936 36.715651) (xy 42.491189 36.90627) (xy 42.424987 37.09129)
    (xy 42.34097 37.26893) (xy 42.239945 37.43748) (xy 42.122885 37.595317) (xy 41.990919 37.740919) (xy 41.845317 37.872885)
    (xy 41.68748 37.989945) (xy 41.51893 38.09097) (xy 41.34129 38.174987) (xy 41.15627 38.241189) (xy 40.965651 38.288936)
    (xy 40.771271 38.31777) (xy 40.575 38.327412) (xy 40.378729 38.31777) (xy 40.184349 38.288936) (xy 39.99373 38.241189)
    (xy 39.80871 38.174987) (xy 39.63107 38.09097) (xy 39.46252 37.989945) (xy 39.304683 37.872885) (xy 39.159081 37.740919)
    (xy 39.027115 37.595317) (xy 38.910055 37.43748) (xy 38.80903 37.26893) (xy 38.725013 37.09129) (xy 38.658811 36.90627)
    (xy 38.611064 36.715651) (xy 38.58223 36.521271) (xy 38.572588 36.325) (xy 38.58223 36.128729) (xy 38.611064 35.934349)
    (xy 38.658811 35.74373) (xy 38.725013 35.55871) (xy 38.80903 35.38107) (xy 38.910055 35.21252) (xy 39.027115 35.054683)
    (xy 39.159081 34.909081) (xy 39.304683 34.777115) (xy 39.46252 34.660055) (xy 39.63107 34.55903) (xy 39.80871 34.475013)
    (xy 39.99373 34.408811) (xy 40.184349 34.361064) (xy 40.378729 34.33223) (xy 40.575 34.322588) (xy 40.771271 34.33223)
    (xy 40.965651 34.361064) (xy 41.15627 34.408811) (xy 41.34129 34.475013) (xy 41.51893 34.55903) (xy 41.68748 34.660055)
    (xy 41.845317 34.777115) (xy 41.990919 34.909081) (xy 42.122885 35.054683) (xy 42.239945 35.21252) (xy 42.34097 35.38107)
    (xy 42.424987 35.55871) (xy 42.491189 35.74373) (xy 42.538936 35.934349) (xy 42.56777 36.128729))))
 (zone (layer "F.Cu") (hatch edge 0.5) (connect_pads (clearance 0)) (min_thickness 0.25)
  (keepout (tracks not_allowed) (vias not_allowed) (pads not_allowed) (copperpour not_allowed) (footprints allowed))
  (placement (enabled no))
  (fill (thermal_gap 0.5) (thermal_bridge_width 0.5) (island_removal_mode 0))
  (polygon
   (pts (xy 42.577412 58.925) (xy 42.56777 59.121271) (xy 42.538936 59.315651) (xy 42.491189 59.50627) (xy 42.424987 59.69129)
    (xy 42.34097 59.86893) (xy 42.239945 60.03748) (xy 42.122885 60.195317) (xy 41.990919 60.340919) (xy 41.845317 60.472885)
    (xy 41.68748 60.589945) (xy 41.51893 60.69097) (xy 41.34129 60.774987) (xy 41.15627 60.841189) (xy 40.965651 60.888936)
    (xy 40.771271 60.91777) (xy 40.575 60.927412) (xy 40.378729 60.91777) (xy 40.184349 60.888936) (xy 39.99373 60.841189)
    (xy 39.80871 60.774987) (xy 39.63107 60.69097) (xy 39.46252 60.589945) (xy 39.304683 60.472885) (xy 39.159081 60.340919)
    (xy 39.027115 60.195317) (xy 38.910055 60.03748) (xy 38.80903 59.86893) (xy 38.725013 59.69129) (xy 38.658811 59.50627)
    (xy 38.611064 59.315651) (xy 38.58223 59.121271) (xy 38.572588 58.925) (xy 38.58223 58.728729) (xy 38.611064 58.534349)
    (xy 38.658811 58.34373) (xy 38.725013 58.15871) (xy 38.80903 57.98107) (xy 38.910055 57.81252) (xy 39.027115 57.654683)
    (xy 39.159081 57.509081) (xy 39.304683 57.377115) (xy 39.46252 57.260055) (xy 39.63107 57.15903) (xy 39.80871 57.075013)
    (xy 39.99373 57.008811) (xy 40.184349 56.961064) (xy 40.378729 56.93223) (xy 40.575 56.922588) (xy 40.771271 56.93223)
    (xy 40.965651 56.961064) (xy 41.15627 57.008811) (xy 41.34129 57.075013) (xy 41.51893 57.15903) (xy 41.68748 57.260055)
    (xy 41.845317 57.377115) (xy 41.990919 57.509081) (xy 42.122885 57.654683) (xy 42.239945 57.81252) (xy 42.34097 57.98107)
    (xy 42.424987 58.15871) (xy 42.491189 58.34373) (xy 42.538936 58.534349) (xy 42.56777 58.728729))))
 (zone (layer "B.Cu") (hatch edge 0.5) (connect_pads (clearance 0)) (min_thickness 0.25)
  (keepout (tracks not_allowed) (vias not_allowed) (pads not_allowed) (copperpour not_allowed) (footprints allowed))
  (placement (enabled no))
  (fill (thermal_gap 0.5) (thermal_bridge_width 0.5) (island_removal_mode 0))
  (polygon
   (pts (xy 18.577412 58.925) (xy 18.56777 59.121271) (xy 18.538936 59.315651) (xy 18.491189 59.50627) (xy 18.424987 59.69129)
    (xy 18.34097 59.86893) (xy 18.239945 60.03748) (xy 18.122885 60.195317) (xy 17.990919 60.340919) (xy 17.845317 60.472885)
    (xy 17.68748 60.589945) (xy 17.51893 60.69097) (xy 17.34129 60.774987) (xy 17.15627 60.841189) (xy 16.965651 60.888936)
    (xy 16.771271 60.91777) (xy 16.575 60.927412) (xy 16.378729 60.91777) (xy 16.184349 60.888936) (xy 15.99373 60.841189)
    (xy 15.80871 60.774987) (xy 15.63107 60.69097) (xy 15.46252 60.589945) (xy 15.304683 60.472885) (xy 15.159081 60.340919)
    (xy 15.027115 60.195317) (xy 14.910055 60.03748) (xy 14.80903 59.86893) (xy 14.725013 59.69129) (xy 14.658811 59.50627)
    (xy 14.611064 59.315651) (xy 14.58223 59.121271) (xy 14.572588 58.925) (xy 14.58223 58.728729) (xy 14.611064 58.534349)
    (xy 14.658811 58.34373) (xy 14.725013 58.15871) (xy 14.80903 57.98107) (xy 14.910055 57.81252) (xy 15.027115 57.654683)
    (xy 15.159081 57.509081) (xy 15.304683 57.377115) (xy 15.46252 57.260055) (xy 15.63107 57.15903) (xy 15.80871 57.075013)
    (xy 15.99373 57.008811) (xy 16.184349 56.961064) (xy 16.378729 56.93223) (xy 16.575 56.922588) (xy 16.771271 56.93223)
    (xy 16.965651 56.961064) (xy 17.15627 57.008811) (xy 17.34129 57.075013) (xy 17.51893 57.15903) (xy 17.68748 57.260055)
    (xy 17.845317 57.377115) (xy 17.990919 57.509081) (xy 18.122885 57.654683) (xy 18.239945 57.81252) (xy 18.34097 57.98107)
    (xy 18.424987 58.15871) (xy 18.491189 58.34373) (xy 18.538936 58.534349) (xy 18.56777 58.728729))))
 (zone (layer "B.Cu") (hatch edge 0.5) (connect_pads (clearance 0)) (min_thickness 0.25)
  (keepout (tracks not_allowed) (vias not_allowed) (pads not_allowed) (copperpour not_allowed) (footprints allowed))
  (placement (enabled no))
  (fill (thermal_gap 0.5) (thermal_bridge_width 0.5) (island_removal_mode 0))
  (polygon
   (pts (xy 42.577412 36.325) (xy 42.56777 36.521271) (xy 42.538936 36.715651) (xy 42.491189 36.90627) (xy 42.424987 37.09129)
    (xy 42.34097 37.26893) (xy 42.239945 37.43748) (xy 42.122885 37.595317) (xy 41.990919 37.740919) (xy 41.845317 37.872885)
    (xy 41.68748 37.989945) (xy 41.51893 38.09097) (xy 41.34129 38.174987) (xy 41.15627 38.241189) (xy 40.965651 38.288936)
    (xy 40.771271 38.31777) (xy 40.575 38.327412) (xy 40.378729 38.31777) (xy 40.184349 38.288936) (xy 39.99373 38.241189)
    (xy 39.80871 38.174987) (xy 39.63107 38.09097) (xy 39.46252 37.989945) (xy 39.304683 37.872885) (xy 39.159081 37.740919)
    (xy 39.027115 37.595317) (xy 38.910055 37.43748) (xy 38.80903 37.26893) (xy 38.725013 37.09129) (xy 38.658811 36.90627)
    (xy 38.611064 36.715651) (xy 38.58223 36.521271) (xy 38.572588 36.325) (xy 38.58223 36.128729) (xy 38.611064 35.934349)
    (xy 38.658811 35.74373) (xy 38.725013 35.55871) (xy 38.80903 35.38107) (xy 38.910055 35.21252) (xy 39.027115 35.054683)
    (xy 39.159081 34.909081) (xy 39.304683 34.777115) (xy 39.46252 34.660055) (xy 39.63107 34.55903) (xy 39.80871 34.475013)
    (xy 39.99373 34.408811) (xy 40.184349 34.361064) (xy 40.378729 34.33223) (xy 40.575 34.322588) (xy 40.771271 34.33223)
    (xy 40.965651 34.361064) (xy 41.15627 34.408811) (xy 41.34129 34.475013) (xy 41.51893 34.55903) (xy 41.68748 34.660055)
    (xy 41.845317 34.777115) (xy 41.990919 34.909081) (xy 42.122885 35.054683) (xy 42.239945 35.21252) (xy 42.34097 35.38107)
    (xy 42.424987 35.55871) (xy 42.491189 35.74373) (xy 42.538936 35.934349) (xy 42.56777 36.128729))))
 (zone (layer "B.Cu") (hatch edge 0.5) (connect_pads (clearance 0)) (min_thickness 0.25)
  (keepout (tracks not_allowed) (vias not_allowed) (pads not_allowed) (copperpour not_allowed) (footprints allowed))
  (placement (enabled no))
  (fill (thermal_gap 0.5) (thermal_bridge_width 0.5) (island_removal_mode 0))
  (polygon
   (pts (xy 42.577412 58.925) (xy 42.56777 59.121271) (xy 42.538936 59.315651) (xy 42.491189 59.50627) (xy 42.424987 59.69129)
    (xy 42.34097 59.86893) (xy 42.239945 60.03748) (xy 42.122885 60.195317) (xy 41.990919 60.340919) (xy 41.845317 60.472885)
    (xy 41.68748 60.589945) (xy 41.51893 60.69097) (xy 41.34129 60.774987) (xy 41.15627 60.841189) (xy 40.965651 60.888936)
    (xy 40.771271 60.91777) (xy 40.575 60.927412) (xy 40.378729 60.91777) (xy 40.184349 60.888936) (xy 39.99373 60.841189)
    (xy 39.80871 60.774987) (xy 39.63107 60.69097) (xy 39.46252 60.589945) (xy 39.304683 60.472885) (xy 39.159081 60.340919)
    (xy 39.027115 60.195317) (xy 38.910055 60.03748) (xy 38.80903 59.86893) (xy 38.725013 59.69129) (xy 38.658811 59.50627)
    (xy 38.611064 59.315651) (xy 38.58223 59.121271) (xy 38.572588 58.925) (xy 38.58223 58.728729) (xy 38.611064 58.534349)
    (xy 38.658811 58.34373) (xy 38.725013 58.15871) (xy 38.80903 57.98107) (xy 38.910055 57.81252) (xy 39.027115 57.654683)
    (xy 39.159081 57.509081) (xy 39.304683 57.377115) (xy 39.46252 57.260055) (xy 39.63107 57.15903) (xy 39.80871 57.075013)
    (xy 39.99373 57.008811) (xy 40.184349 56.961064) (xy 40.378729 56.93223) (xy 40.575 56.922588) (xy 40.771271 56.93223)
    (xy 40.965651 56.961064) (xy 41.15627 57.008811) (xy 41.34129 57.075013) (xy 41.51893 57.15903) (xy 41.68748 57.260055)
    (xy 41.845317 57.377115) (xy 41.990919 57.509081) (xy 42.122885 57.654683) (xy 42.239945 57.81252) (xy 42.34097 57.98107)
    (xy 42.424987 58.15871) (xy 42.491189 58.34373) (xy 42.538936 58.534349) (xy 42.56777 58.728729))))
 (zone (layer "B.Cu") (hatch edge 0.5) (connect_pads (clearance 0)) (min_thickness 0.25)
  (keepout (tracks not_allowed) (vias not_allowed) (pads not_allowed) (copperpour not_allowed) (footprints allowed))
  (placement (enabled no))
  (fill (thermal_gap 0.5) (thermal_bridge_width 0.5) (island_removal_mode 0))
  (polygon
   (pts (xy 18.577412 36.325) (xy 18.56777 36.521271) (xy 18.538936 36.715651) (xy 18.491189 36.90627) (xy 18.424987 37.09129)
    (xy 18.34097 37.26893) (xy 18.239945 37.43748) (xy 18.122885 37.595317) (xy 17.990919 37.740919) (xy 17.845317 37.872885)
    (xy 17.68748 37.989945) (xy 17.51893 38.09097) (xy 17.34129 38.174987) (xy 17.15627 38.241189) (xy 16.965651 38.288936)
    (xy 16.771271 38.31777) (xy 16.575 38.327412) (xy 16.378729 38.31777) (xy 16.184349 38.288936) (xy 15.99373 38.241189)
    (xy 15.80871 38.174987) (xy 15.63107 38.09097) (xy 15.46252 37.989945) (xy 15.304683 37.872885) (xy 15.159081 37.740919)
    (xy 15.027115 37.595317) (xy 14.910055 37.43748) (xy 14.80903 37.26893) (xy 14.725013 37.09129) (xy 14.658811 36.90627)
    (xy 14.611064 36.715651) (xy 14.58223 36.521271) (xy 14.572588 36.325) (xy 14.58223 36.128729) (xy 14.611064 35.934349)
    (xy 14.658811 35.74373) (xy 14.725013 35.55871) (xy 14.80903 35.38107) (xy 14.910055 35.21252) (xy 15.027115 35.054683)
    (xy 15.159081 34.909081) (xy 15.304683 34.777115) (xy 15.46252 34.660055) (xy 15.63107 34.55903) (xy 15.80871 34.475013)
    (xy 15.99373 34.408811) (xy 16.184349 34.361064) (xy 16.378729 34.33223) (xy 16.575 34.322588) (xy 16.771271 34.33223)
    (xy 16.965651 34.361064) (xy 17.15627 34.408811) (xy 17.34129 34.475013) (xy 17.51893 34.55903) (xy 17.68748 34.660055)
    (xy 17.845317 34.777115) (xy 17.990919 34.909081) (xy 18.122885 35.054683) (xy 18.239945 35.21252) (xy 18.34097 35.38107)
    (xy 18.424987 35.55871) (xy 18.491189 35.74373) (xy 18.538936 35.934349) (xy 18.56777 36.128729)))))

